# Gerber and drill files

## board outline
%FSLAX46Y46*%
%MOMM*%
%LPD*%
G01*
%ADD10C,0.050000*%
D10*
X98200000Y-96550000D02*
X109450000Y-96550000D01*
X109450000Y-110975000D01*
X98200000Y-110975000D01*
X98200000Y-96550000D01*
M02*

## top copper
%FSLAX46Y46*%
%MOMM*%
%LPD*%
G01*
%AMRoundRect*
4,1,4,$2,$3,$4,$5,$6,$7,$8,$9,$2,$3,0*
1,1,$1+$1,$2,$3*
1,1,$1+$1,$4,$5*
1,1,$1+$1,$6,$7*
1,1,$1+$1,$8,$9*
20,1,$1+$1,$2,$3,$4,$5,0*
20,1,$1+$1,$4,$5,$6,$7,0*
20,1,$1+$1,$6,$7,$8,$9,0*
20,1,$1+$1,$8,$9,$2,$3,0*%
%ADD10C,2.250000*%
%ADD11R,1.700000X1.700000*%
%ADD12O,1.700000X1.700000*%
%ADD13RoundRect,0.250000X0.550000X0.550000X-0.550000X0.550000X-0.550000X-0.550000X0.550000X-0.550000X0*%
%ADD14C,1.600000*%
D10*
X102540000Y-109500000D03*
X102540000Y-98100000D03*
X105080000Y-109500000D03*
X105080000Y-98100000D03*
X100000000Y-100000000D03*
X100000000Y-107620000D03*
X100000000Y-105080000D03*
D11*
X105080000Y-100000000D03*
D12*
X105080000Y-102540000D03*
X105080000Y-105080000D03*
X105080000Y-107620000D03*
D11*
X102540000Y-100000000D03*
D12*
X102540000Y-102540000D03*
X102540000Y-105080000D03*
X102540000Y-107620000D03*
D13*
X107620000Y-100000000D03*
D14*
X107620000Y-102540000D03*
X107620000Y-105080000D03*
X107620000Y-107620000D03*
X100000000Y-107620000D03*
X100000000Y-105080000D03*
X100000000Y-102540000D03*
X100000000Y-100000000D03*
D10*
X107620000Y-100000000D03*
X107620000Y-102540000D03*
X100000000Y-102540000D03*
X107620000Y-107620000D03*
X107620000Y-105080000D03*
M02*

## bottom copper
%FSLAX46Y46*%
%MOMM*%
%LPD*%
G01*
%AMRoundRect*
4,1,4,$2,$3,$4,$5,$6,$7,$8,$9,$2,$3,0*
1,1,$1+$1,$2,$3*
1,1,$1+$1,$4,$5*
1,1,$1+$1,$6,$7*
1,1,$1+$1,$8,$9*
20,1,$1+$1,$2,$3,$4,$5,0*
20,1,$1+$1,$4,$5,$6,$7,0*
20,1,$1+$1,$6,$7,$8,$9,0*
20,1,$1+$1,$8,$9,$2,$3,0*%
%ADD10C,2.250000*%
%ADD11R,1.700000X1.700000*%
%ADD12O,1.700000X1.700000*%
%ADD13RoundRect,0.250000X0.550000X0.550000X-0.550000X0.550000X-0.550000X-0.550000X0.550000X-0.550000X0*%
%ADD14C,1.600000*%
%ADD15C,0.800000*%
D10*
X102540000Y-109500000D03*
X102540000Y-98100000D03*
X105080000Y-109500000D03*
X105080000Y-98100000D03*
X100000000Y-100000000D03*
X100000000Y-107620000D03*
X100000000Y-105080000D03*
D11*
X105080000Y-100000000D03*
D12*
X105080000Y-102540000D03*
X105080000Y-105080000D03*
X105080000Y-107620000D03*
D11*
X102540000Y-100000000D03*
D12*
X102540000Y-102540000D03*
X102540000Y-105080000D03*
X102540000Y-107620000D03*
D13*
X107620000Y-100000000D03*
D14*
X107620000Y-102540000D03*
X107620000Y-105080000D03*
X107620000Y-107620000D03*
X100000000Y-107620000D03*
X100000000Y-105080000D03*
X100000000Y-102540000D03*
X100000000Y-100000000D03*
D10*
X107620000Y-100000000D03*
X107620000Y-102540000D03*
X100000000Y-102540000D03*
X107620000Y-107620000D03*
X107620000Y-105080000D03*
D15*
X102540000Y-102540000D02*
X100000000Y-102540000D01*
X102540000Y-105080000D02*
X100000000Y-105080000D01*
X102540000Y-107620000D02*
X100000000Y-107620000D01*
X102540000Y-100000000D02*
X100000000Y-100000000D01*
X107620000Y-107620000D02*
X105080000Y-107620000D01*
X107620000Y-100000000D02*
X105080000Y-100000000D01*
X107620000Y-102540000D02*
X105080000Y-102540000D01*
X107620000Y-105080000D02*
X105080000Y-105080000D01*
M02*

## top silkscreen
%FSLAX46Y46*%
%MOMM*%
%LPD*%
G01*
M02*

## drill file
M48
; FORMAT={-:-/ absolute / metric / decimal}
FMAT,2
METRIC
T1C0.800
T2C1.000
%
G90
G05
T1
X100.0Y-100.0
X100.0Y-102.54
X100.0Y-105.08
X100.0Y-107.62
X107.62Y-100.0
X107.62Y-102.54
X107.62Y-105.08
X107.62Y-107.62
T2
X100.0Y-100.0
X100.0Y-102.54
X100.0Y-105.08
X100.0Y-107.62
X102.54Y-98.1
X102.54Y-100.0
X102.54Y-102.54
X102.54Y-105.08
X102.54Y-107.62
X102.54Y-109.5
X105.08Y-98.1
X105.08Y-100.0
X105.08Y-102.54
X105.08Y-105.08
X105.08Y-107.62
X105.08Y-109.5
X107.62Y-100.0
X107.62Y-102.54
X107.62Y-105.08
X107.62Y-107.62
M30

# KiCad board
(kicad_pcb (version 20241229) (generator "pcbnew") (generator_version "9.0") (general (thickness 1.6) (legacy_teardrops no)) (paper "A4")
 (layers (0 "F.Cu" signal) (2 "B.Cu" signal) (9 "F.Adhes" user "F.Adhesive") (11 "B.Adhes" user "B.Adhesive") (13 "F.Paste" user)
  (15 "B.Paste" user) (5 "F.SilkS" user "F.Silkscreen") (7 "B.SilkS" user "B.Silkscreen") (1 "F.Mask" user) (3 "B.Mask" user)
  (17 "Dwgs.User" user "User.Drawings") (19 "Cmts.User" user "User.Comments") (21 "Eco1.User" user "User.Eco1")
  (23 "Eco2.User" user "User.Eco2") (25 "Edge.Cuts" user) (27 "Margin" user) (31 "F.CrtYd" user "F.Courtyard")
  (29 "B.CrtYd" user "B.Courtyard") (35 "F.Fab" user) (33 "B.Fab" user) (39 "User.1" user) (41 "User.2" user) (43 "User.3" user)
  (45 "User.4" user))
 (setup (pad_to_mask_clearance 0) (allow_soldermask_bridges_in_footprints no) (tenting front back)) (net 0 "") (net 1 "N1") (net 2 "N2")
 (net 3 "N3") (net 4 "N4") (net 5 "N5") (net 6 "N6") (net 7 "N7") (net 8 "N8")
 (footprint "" (layer "F.Cu") (at 102.485 110.405)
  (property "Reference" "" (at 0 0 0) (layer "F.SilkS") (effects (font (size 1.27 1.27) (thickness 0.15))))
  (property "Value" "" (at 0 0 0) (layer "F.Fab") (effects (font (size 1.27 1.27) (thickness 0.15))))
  (pad "1" thru_hole circle (at 0.055 -0.905 180) (size 2.25 2.25) (drill 1) (layers "*.Cu" "*.Mask") (remove_unused_layers no)))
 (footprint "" (layer "F.Cu") (at 102.55 98.125)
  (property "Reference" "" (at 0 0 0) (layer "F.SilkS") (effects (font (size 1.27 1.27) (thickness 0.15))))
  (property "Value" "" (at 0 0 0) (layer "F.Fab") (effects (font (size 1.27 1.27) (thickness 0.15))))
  (pad "1" thru_hole circle (at -0.01 -0.025 180) (size 2.25 2.25) (drill 1) (layers "*.Cu" "*.Mask") (remove_unused_layers no)))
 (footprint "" (layer "F.Cu") (at 105.04 109.575)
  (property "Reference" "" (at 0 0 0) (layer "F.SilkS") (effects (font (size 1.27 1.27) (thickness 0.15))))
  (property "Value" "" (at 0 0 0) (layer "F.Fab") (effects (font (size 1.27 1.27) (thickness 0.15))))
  (pad "1" thru_hole circle (at 0.04 -0.075 180) (size 2.25 2.25) (drill 1) (layers "*.Cu" "*.Mask") (remove_unused_layers no)))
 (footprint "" (layer "F.Cu") (at 105.05 97.8)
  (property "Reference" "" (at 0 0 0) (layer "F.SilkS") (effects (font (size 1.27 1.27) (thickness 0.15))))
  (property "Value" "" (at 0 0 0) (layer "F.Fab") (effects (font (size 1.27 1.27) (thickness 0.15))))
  (pad "1" thru_hole circle (at 0.03 0.3 180) (size 2.25 2.25) (drill 1) (layers "*.Cu" "*.Mask") (remove_unused_layers no)))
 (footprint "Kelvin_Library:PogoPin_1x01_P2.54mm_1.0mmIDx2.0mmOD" (layer "B.Cu") (at 100 100 180)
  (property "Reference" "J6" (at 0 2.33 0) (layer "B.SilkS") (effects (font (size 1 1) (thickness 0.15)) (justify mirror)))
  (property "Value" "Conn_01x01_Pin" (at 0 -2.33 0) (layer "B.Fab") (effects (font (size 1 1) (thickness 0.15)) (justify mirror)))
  (pad "1" thru_hole circle (at 0 0 180) (size 2.25 2.25) (drill 1) (layers "*.Cu" "*.Mask") (remove_unused_layers no) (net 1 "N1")))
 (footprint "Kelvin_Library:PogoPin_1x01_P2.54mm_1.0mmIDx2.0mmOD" (layer "B.Cu") (at 100 107.62 180)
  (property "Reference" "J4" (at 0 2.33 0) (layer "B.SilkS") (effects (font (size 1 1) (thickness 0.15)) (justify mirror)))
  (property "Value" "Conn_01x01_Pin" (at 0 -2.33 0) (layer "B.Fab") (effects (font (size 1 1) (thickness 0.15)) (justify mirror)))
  (pad "1" thru_hole circle (at 0 0 180) (size 2.25 2.25) (drill 1) (layers "*.Cu" "*.Mask") (remove_unused_layers no) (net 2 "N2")))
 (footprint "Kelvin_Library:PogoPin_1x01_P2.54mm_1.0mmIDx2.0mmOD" (layer "B.Cu") (at 100 105.08 180)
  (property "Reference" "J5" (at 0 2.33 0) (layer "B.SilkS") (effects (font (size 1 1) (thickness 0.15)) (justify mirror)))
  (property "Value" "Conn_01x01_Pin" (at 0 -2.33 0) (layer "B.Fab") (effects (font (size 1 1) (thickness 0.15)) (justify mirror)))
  (pad "1" thru_hole circle (at 0 0 180) (size 2.25 2.25) (drill 1) (layers "*.Cu" "*.Mask") (remove_unused_layers no) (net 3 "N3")))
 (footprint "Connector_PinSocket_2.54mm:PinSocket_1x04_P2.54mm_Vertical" (layer "B.Cu") (at 105.08 100 180)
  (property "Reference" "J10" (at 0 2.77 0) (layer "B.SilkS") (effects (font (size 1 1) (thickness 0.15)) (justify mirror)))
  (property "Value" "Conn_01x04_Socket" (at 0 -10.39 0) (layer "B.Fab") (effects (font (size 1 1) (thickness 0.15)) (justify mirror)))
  (pad "1" thru_hole rect (at 0 0 180) (size 1.7 1.7) (drill 1) (layers "*.Cu" "*.Mask") (remove_unused_layers no) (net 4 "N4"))
  (pad "2" thru_hole oval (at 0 -2.54 180) (size 1.7 1.7) (drill 1) (layers "*.Cu" "*.Mask") (remove_unused_layers no) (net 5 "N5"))
  (pad "3" thru_hole oval (at 0 -5.08 180) (size 1.7 1.7) (drill 1) (layers "*.Cu" "*.Mask") (remove_unused_layers no) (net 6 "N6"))
  (pad "4" thru_hole oval (at 0 -7.62 180) (size 1.7 1.7) (drill 1) (layers "*.Cu" "*.Mask") (remove_unused_layers no) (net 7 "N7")))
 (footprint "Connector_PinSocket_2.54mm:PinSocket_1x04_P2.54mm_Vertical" (layer "B.Cu") (at 102.54 100 180)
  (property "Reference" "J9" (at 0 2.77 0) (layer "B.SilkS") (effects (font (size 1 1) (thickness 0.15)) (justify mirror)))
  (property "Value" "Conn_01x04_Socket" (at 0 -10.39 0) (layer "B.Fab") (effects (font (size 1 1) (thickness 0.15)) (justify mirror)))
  (pad "1" thru_hole rect (at 0 0 180) (size 1.7 1.7) (drill 1) (layers "*.Cu" "*.Mask") (remove_unused_layers no) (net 1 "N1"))
  (pad "2" thru_hole oval (at 0 -2.54 180) (size 1.7 1.7) (drill 1) (layers "*.Cu" "*.Mask") (remove_unused_layers no) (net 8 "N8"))
  (pad "3" thru_hole oval (at 0 -5.08 180) (size 1.7 1.7) (drill 1) (layers "*.Cu" "*.Mask") (remove_unused_layers no) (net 3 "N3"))
  (pad "4" thru_hole oval (at 0 -7.62 180) (size 1.7 1.7) (drill 1) (layers "*.Cu" "*.Mask") (remove_unused_layers no) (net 2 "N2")))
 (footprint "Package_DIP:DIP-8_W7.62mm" (layer "B.Cu") (at 107.62 100 180)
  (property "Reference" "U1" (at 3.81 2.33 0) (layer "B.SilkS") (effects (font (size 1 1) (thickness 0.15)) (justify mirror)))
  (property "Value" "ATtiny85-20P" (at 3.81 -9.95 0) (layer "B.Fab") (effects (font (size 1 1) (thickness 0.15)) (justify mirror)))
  (pad "1" thru_hole roundrect (at 0 0 180) (size 1.6 1.6) (drill 0.8) (layers "*.Cu" "*.Mask") (remove_unused_layers no)
   (roundrect_rratio 0.15625) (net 4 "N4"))
  (pad "2" thru_hole circle (at 0 -2.54 180) (size 1.6 1.6) (drill 0.8) (layers "*.Cu" "*.Mask") (remove_unused_layers no) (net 5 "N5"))
  (pad "3" thru_hole circle (at 0 -5.08 180) (size 1.6 1.6) (drill 0.8) (layers "*.Cu" "*.Mask") (remove_unused_layers no) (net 6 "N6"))
  (pad "4" thru_hole circle (at 0 -7.62 180) (size 1.6 1.6) (drill 0.8) (layers "*.Cu" "*.Mask") (remove_unused_layers no) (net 7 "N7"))
  (pad "5" thru_hole circle (at 7.62 -7.62 180) (size 1.6 1.6) (drill 0.8) (layers "*.Cu" "*.Mask") (remove_unused_layers no) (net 2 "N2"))
  (pad "6" thru_hole circle (at 7.62 -5.08 180) (size 1.6 1.6) (drill 0.8) (layers "*.Cu" "*.Mask") (remove_unused_layers no) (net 3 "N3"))
  (pad "7" thru_hole circle (at 7.62 -2.54 180) (size 1.6 1.6) (drill 0.8) (layers "*.Cu" "*.Mask") (remove_unused_layers no) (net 8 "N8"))
  (pad "8" thru_hole circle (at 7.62 0 180) (size 1.6 1.6) (drill 0.8) (layers "*.Cu" "*.Mask") (remove_unused_layers no) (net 1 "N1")))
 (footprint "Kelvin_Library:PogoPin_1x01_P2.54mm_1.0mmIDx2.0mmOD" (layer "B.Cu") (at 107.62 100 180)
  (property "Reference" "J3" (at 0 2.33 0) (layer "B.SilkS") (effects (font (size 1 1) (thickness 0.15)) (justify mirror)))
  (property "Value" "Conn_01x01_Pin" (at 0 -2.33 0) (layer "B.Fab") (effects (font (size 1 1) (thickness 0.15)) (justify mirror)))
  (pad "1" thru_hole circle (at 0 0 180) (size 2.25 2.25) (drill 1) (layers "*.Cu" "*.Mask") (remove_unused_layers no) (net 4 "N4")))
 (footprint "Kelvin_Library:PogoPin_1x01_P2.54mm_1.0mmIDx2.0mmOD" (layer "B.Cu") (at 107.62 102.54 180)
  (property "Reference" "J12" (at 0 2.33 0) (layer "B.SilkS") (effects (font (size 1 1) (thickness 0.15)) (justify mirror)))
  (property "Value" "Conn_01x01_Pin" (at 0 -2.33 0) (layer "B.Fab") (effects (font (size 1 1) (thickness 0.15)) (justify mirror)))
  (pad "1" thru_hole circle (at 0 0 180) (size 2.25 2.25) (drill 1) (layers "*.Cu" "*.Mask") (remove_unused_layers no) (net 5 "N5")))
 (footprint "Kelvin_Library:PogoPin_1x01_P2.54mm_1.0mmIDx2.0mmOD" (layer "B.Cu") (at 100 102.54 180)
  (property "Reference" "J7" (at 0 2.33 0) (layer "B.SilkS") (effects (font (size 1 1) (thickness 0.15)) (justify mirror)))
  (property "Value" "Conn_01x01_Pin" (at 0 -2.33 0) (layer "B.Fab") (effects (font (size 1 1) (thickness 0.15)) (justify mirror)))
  (pad "1" thru_hole circle (at 0 0 180) (size 2.25 2.25) (drill 1) (layers "*.Cu" "*.Mask") (remove_unused_layers no) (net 8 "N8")))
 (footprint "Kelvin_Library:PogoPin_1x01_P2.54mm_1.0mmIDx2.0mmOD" (layer "B.Cu") (at 107.62 107.62 180)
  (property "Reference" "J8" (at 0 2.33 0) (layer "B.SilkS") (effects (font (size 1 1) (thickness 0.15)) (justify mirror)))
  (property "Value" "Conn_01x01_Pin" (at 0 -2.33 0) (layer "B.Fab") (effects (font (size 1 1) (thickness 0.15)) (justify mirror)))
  (pad "1" thru_hole circle (at 0 0 180) (size 2.25 2.25) (drill 1) (layers "*.Cu" "*.Mask") (remove_unused_layers no) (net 7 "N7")))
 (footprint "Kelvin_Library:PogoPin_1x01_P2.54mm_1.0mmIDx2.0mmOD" (layer "B.Cu") (at 107.62 105.08 180)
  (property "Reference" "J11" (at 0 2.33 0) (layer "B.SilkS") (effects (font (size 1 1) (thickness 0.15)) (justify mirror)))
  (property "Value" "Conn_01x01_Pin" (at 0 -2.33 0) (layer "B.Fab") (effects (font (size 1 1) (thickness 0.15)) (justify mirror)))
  (pad "1" thru_hole circle (at 0 0 180) (size 2.25 2.25) (drill 1) (layers "*.Cu" "*.Mask") (remove_unused_layers no) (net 6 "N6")))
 (gr_rect (start 98.2 96.55) (end 109.45 110.975) (stroke (width 0.05) (type default)) (fill no) (layer "Edge.Cuts"))
 (segment (start 102.54 102.54) (end 100 102.54) (width 0.8) (layer "B.Cu") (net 8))
 (segment (start 102.54 105.08) (end 100 105.08) (width 0.8) (layer "B.Cu") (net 3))
 (segment (start 102.54 107.62) (end 100 107.62) (width 0.8) (layer "B.Cu") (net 2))
 (segment (start 102.54 100) (end 100 100) (width 0.8) (layer "B.Cu") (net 1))
 (segment (start 107.62 107.62) (end 105.08 107.62) (width 0.8) (layer "B.Cu") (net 7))
 (segment (start 107.62 100) (end 105.08 100) (width 0.8) (layer "B.Cu") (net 4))
 (segment (start 107.62 102.54) (end 105.08 102.54) (width 0.8) (layer "B.Cu") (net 5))
 (segment (start 107.62 105.08) (end 105.08 105.08) (width 0.8) (layer "B.Cu") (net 6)))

